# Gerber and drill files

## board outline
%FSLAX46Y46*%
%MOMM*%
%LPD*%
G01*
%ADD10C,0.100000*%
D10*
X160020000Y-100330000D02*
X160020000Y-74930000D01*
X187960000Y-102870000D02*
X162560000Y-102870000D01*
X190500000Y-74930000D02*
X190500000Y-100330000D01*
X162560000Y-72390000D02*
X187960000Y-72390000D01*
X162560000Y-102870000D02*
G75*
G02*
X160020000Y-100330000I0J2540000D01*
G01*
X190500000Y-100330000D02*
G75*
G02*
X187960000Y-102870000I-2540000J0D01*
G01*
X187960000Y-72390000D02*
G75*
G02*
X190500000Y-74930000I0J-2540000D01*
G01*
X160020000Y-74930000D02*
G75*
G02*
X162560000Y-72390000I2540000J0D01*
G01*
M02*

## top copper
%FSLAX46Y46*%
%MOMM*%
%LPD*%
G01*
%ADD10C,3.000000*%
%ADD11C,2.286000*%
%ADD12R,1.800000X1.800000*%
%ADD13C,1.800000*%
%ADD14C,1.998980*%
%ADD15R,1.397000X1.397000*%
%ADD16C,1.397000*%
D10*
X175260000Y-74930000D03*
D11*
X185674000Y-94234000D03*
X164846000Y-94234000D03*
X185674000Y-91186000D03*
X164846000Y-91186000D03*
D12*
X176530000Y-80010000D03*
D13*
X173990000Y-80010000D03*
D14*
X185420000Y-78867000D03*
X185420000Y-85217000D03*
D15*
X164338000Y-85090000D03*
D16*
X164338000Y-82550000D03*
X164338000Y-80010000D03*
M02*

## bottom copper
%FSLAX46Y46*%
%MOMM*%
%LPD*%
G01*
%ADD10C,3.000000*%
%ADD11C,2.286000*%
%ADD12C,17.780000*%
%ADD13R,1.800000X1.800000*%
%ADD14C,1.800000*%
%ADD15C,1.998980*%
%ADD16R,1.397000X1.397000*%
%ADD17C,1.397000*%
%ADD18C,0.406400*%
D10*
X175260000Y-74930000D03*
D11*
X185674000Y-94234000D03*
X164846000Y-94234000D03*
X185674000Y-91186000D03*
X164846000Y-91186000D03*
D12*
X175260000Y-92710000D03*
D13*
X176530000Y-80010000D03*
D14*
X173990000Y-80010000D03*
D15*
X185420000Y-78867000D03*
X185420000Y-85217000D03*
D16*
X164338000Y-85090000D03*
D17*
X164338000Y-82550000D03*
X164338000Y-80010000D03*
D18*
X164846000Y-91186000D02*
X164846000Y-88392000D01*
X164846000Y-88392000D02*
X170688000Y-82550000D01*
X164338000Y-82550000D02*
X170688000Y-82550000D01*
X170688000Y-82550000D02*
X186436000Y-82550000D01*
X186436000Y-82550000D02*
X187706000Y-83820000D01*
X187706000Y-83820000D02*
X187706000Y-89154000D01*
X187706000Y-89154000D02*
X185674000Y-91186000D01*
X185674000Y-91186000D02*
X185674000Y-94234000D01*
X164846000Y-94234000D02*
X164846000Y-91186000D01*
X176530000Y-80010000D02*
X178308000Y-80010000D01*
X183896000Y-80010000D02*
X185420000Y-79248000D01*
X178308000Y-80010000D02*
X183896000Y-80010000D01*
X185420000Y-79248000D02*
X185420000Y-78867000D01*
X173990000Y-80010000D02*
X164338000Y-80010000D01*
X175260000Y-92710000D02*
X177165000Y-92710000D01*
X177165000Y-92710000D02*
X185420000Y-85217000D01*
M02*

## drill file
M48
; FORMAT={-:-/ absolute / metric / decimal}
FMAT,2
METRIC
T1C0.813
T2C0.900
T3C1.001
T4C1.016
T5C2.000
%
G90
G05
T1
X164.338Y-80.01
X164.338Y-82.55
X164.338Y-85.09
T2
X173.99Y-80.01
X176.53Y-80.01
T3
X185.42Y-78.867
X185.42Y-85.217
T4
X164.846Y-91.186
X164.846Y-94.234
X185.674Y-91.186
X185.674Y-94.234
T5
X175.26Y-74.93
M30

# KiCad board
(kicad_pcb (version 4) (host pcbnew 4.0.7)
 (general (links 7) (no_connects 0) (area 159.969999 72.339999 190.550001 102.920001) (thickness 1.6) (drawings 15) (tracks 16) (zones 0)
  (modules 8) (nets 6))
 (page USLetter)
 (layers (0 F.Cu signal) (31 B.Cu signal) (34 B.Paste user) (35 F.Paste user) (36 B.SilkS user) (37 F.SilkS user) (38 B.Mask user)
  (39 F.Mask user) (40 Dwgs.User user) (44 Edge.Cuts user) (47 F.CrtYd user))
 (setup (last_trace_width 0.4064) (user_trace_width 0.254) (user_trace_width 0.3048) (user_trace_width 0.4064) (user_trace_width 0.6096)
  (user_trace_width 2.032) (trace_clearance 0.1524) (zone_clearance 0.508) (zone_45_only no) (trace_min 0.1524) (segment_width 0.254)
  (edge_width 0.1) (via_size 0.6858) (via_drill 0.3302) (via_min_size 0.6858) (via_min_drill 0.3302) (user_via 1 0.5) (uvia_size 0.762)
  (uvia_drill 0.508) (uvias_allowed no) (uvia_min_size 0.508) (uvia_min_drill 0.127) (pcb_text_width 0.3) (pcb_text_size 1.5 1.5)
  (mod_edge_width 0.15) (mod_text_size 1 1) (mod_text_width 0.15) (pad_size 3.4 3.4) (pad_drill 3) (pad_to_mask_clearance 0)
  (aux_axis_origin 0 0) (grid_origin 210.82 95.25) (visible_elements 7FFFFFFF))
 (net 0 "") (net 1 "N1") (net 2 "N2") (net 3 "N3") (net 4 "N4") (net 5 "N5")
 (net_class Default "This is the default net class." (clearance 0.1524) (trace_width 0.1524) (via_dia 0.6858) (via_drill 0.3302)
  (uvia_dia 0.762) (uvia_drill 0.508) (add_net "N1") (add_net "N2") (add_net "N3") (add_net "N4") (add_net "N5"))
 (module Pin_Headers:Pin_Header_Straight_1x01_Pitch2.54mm (layer F.Cu) (at 175.26 74.93)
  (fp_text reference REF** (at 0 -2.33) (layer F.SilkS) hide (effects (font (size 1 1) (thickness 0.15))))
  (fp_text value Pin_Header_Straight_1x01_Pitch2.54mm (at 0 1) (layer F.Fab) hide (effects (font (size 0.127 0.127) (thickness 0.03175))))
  (pad 1 thru_hole circle (at 0 0) (size 3 3) (drill 2) (layers *.Cu *.Mask)))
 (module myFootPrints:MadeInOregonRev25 (layer F.Cu) (at 169.672 81.534)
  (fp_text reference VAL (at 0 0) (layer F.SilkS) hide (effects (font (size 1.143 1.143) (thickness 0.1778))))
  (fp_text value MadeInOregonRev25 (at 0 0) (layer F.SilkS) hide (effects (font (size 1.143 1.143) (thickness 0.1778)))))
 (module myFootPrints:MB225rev (layer F.Cu) (at 181.102 81.534)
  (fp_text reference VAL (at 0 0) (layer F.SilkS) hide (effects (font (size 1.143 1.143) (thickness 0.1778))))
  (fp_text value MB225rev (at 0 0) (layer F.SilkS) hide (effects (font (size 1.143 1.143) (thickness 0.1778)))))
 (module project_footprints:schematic (layer F.Cu) (at 174.498 90.678)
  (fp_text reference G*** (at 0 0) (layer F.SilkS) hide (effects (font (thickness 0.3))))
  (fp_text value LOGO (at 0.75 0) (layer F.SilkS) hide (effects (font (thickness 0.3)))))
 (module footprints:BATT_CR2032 (layer B.Cu) (at 175.26 92.71 180)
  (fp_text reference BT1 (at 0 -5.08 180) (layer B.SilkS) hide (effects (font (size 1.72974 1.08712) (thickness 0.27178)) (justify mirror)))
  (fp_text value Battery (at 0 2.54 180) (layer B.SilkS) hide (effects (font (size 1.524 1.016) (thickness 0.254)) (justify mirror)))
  (pad 1 thru_hole circle (at -10.414 -1.524 180) (size 2.286 2.286) (drill 1.016) (layers *.Cu *.Mask B.SilkS) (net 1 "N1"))
  (pad 1 thru_hole circle (at 10.414 -1.524 180) (size 2.286 2.286) (drill 1.016) (layers *.Cu *.Mask B.SilkS) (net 1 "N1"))
  (pad 1 thru_hole circle (at -10.414 1.524 180) (size 2.286 2.286) (drill 1.016) (layers *.Cu *.Mask B.SilkS) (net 1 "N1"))
  (pad 1 thru_hole circle (at 10.414 1.524 180) (size 2.286 2.286) (drill 1.016) (layers *.Cu *.Mask B.SilkS) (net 1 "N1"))
  (pad 2 smd circle (at 0 0 180) (size 17.78 17.78) (layers B.Cu B.Paste B.Mask) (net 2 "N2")))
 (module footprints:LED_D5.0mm (layer F.Cu) (at 176.53 80.01 180)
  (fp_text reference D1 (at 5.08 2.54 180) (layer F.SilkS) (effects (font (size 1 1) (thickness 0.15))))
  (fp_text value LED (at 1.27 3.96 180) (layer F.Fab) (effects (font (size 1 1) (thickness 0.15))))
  (pad 1 thru_hole rect (at 0 0 180) (size 1.8 1.8) (drill 0.9) (layers *.Cu *.Mask) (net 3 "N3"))
  (pad 2 thru_hole circle (at 2.54 0 180) (size 1.8 1.8) (drill 0.9) (layers *.Cu *.Mask) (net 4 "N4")))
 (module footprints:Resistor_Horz (layer F.Cu) (at 185.42 82.042 270)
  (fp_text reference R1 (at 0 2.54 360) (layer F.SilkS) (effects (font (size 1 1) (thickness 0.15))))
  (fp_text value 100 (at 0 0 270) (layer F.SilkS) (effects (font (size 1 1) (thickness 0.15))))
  (pad 1 thru_hole circle (at -3.175 0 270) (size 1.99898 1.99898) (drill 1.00076) (layers *.Cu *.SilkS *.Mask) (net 3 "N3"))
  (pad 2 thru_hole circle (at 3.175 0 270) (size 1.99898 1.99898) (drill 1.00076) (layers *.Cu *.SilkS *.Mask) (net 2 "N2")))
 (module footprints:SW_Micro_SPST (layer F.Cu) (at 164.338 82.55 90)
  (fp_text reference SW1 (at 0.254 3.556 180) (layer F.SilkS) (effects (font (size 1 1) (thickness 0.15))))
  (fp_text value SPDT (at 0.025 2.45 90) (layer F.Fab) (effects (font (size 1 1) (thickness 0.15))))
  (pad 1 thru_hole rect (at -2.54 0 90) (size 1.397 1.397) (drill 0.8128) (layers *.Cu *.Mask F.SilkS) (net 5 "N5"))
  (pad 2 thru_hole circle (at 0 0 90) (size 1.397 1.397) (drill 0.8128) (layers *.Cu *.Mask F.SilkS) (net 1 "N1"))
  (pad 3 thru_hole circle (at 2.54 0 90) (size 1.397 1.397) (drill 0.8128) (layers *.Cu *.Mask F.SilkS) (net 4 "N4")))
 (gr_line (start 160.02 100.33) (end 160.02 74.93) (angle 90) (layer Edge.Cuts) (width 0.1))
 (gr_line (start 187.96 102.87) (end 162.56 102.87) (angle 90) (layer Edge.Cuts) (width 0.1))
 (gr_line (start 190.5 74.93) (end 190.5 100.33) (angle 90) (layer Edge.Cuts) (width 0.1))
 (gr_line (start 162.56 72.39) (end 187.96 72.39) (angle 90) (layer Edge.Cuts) (width 0.1))
 (gr_arc (start 162.56 100.33) (end 162.56 102.87) (angle 90) (layer Edge.Cuts) (width 0.1))
 (gr_arc (start 187.96 100.33) (end 190.5 100.33) (angle 90) (layer Edge.Cuts) (width 0.1))
 (gr_arc (start 187.96 74.93) (end 187.96 72.39) (angle 90) (layer Edge.Cuts) (width 0.1))
 (gr_arc (start 162.56 74.93) (end 160.02 74.93) (angle 90) (layer Edge.Cuts) (width 0.1))
 (segment (start 164.846 91.186) (end 164.846 88.392) (width 0.4064) (layer B.Cu) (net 1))
 (segment (start 164.846 88.392) (end 170.688 82.55) (width 0.4064) (layer B.Cu) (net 1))
 (segment (start 164.338 82.55) (end 170.688 82.55) (width 0.4064) (layer B.Cu) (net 1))
 (segment (start 170.688 82.55) (end 186.436 82.55) (width 0.4064) (layer B.Cu) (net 1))
 (segment (start 186.436 82.55) (end 187.706 83.82) (width 0.4064) (layer B.Cu) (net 1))
 (segment (start 187.706 83.82) (end 187.706 89.154) (width 0.4064) (layer B.Cu) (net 1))
 (segment (start 187.706 89.154) (end 185.674 91.186) (width 0.4064) (layer B.Cu) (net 1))
 (segment (start 185.674 91.186) (end 185.674 94.234) (width 0.4064) (layer B.Cu) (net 1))
 (segment (start 164.846 94.234) (end 164.846 91.186) (width 0.4064) (layer B.Cu) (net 1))
 (segment (start 176.53 80.01) (end 178.308 80.01) (width 0.4064) (layer B.Cu) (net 3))
 (segment (start 183.896 80.01) (end 185.42 79.248) (width 0.4064) (layer B.Cu) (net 3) (status 20))
 (segment (start 178.308 80.01) (end 183.896 80.01) (width 0.4064) (layer B.Cu) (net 3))
 (segment (start 185.42 79.248) (end 185.42 78.867) (width 0.4064) (layer B.Cu) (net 3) (status 30))
 (segment (start 173.99 80.01) (end 164.338 80.01) (width 0.4064) (layer B.Cu) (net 4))
 (segment (start 175.26 92.71) (end 177.165 92.71) (width 0.4064) (layer B.Cu) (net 2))
 (segment (start 177.165 92.71) (end 185.42 85.217) (width 0.4064) (layer B.Cu) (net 2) (status 20)))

